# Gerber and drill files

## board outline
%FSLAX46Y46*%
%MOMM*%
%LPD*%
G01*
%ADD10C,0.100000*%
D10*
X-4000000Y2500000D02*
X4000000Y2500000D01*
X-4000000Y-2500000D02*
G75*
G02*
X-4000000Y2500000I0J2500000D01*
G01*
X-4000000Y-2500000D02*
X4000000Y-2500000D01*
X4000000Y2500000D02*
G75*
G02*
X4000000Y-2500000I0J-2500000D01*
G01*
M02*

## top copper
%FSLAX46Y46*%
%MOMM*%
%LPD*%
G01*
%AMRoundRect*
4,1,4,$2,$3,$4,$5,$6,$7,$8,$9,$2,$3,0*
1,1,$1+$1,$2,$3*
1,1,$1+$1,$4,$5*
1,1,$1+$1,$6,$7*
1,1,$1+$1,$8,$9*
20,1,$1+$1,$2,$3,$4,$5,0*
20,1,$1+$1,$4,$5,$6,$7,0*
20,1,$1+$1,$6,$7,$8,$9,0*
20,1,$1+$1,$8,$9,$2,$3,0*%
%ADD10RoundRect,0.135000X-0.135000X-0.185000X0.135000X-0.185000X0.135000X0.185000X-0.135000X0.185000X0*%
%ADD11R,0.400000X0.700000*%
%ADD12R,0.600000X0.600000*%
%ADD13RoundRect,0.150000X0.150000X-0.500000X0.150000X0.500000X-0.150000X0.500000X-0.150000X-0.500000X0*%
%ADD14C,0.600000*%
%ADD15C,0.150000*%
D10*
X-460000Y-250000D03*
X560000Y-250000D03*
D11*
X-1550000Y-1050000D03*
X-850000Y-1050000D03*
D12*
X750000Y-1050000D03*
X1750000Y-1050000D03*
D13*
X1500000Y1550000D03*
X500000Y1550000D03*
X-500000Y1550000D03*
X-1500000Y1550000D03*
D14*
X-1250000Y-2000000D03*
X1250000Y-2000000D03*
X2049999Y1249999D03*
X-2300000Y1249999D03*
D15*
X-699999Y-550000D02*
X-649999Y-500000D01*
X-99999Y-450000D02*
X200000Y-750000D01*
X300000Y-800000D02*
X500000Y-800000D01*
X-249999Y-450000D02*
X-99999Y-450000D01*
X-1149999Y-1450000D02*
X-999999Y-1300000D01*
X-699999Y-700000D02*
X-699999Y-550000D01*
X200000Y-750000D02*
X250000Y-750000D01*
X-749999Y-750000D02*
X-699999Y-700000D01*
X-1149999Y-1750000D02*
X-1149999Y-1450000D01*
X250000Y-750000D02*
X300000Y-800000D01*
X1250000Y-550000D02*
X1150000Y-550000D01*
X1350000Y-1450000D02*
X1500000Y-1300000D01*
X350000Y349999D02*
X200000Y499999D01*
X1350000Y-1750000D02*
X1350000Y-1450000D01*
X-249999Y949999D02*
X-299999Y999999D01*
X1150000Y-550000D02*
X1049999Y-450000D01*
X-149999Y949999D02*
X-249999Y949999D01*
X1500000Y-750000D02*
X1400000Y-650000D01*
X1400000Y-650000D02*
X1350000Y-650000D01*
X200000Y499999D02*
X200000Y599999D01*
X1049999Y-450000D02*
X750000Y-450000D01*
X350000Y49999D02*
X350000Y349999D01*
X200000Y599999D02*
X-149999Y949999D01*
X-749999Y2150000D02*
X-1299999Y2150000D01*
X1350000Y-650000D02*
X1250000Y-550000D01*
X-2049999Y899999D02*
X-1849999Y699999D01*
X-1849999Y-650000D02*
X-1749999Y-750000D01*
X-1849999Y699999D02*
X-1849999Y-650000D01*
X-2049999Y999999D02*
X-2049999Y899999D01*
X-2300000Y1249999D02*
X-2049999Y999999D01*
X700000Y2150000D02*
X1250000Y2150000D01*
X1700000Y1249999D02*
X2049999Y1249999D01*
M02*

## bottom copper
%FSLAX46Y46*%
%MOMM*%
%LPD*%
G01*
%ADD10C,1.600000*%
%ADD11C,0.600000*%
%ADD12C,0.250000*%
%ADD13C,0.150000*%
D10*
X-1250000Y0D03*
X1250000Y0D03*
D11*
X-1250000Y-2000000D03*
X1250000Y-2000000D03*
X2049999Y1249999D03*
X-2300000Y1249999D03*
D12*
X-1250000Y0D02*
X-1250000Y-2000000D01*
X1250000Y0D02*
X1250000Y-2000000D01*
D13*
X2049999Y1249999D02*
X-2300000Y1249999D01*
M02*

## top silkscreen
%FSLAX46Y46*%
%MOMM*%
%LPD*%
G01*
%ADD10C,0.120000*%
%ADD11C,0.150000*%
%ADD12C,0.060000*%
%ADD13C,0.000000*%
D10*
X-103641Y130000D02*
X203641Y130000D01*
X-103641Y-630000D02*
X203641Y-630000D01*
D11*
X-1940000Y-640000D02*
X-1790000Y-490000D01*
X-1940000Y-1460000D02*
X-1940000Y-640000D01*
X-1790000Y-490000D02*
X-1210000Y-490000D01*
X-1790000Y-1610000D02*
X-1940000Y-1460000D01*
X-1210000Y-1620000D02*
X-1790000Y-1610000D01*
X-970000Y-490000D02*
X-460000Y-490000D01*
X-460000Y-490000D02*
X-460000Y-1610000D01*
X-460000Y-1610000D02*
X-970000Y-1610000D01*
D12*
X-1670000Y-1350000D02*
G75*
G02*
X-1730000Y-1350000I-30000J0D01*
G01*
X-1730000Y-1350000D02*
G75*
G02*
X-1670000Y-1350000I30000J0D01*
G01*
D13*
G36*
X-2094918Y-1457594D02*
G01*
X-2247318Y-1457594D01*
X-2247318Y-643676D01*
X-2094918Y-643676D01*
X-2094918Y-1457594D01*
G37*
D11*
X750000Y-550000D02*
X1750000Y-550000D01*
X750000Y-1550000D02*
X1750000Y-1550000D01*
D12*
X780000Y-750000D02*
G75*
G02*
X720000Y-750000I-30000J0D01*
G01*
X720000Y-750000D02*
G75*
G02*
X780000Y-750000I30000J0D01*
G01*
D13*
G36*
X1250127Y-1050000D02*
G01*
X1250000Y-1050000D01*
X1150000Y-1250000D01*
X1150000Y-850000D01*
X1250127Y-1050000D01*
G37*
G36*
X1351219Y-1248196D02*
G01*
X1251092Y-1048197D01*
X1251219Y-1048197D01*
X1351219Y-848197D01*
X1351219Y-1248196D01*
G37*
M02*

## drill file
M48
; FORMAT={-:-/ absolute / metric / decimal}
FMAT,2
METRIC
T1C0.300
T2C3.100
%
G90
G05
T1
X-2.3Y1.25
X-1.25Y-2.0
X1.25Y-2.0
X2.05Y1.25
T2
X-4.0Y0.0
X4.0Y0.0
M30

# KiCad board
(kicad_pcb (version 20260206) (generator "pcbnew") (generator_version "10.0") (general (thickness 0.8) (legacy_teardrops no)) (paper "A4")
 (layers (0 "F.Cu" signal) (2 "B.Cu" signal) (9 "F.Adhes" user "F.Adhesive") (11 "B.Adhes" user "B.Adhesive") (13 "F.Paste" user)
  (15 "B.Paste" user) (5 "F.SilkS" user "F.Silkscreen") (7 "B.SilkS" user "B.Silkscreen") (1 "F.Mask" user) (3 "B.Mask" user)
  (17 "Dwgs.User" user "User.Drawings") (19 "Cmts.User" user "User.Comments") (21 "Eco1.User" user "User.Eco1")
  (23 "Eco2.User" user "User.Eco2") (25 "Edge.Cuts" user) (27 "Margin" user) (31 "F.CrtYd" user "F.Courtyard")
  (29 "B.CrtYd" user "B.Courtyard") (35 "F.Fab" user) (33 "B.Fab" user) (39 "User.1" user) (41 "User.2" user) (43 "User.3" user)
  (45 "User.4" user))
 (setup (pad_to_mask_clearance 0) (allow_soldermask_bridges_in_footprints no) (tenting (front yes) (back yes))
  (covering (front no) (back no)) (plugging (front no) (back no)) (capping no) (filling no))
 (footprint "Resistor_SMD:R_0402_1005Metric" (layer "F.Cu") (at 0.05 0.25)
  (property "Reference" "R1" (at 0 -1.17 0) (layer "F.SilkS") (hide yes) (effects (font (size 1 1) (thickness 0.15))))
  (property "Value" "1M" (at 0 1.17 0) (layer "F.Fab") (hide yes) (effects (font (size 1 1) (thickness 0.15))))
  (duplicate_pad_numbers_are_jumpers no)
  (fp_line (start -0.153641 -0.38) (end 0.153641 -0.38) (stroke (width 0.12) (type solid)) (layer "F.SilkS"))
  (fp_line (start -0.153641 0.38) (end 0.153641 0.38) (stroke (width 0.12) (type solid)) (layer "F.SilkS"))
  (pad "1" smd roundrect (at -0.51 0) (size 0.54 0.64) (layers "F.Cu" "F.Mask" "F.Paste") (roundrect_rratio 0.25) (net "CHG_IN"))
  (pad "2" smd roundrect (at 0.51 0) (size 0.54 0.64) (layers "F.Cu" "F.Mask" "F.Paste") (roundrect_rratio 0.25) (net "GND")))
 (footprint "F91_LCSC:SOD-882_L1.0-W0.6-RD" (layer "F.Cu") (at -1.2 1.05)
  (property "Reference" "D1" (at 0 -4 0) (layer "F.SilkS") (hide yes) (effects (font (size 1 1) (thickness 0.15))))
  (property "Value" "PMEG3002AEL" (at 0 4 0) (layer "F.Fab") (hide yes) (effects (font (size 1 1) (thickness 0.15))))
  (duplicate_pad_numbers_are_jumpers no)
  (fp_line (start -0.74 -0.41) (end -0.59 -0.56) (stroke (width 0.15) (type solid)) (layer "F.SilkS"))
  (fp_line (start -0.74 0.41) (end -0.74 -0.41) (stroke (width 0.15) (type solid)) (layer "F.SilkS"))
  (fp_line (start -0.59 -0.56) (end -0.01 -0.56) (stroke (width 0.15) (type solid)) (layer "F.SilkS"))
  (fp_line (start -0.59 0.56) (end -0.74 0.41) (stroke (width 0.15) (type solid)) (layer "F.SilkS"))
  (fp_line (start -0.01 0.57) (end -0.59 0.56) (stroke (width 0.15) (type solid)) (layer "F.SilkS"))
  (fp_line (start 0.23 -0.56) (end 0.74 -0.56) (stroke (width 0.15) (type solid)) (layer "F.SilkS"))
  (fp_line (start 0.74 -0.56) (end 0.74 0.56) (stroke (width 0.15) (type solid)) (layer "F.SilkS"))
  (fp_line (start 0.74 0.56) (end 0.23 0.56) (stroke (width 0.15) (type solid)) (layer "F.SilkS"))
  (fp_circle (center -0.5 0.3) (end -0.47 0.3) (stroke (width 0.06) (type solid)) (fill no) (layer "F.SilkS"))
  (fp_poly
   (pts (xy -0.894918 0.407594) (xy -0.894918 -0.406324) (xy -1.047318 -0.406324) (xy -1.047318 0.407594) (xy -0.894918 0.407594))
   (stroke (width 0) (type solid)) (fill yes) (layer "F.SilkS"))
  (pad "1" smd rect (at -0.35 0) (size 0.4 0.7) (layers "F.Cu" "F.Mask" "F.Paste") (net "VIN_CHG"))
  (pad "2" smd rect (at 0.35 0) (size 0.4 0.7) (layers "F.Cu" "F.Mask" "F.Paste") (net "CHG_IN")))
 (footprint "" (layer "F.Cu") (at 0 0)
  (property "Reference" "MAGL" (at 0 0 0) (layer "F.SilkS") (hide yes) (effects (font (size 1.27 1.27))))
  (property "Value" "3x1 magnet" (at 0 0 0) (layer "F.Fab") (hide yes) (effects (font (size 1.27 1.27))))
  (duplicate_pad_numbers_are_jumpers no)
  (pad "" np_thru_hole circle (at -4 0) (size 3.1 3.1) (drill 3.1) (layers "*.Cu")))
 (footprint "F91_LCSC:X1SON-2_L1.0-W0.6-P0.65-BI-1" (layer "F.Cu") (at 1.25 1.05)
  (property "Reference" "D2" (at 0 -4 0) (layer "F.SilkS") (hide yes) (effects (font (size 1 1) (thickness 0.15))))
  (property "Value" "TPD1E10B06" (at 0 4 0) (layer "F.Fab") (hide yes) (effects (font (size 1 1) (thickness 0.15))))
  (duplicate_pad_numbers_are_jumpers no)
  (fp_line (start -0.5 -0.5) (end 0.5 -0.5) (stroke (width 0.15) (type solid)) (layer "F.SilkS"))
  (fp_line (start -0.5 0.5) (end 0.5 0.5) (stroke (width 0.15) (type solid)) (layer "F.SilkS"))
  (fp_circle (center -0.5 -0.3) (end -0.47 -0.3) (stroke (width 0.06) (type solid)) (fill no) (layer "F.SilkS"))
  (fp_poly
   (pts (xy -0.1 -0.2) (xy -0.1 0.2) (xy 0 0) (xy 0.000127 0) (xy -0.1 -0.2)) (stroke (width 0) (type solid)) (fill yes) (layer "F.SilkS"))
  (fp_poly
   (pts (xy 0.101219 0.198196) (xy 0.101219 -0.201803) (xy 0.001219 -0.001803) (xy 0.001092 -0.001803) (xy 0.101219 0.198196))
   (stroke (width 0) (type solid)) (fill yes) (layer "F.SilkS"))
  (pad "1" smd rect (at -0.5 0) (size 0.6 0.6) (layers "F.Cu" "F.Mask" "F.Paste") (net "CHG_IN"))
  (pad "2" smd rect (at 0.5 0) (size 0.6 0.6) (layers "F.Cu" "F.Mask" "F.Paste") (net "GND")))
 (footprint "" (layer "F.Cu") (at 0 0)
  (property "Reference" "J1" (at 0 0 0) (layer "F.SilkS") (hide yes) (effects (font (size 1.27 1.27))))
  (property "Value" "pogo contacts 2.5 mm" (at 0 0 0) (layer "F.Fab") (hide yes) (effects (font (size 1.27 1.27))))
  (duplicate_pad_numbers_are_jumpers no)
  (pad "1" smd circle (at -1.25 0) (size 1.6 1.6) (layers "B.Cu" "B.Mask") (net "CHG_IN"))
  (pad "2" smd circle (at 1.25 0) (size 1.6 1.6) (layers "B.Cu" "B.Mask") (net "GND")))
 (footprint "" (layer "F.Cu") (at 0 0)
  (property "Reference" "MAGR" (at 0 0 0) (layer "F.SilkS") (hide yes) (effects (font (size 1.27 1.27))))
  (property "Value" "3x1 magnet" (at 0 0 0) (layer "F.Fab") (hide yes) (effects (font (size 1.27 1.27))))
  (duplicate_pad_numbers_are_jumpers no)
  (pad "" np_thru_hole circle (at 4 0) (size 3.1 3.1) (drill 3.1) (layers "*.Cu")))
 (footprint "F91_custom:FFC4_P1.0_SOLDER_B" (layer "B.Cu") (at 0 -1.55 90)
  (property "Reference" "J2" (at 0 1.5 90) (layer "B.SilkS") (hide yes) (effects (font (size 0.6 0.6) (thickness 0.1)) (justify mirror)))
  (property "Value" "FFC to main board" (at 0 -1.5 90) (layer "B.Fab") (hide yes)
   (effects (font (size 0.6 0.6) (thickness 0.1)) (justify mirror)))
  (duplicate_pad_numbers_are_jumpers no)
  (pad "1" smd roundrect (at 0 1.5 90) (size 1.3 0.6) (layers "F.Cu" "F.Mask") (roundrect_rratio 0.25) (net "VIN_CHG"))
  (pad "2" smd roundrect (at 0 0.5 90) (size 1.3 0.6) (layers "F.Cu" "F.Mask") (roundrect_rratio 0.25) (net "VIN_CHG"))
  (pad "3" smd roundrect (at 0 -0.5 90) (size 1.3 0.6) (layers "F.Cu" "F.Mask") (roundrect_rratio 0.25) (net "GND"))
  (pad "4" smd roundrect (at 0 -1.5 90) (size 1.3 0.6) (layers "F.Cu" "F.Mask") (roundrect_rratio 0.25) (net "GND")))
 (gr_line (start -4 -2.5) (end 4 -2.5) (stroke (width 0.1) (type default)) (layer "Edge.Cuts"))
 (gr_arc (start -4 2.5) (mid -6.5 0) (end -4 -2.5) (stroke (width 0.1) (type default)) (layer "Edge.Cuts"))
 (gr_line (start -4 2.5) (end 4 2.5) (stroke (width 0.1) (type default)) (layer "Edge.Cuts"))
 (gr_arc (start 4 -2.5) (mid 6.5 0) (end 4 2.5) (stroke (width 0.1) (type default)) (layer "Edge.Cuts"))
 (segment (start -0.699999 0.55) (end -0.649999 0.5) (width 0.15) (layer "F.Cu") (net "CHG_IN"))
 (segment (start -0.099999 0.45) (end 0.2 0.75) (width 0.15) (layer "F.Cu") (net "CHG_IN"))
 (segment (start 0.3 0.8) (end 0.5 0.8) (width 0.15) (layer "F.Cu") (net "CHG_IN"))
 (segment (start -0.249999 0.45) (end -0.099999 0.45) (width 0.15) (layer "F.Cu") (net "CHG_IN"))
 (segment (start -1.149999 1.45) (end -0.999999 1.3) (width 0.15) (layer "F.Cu") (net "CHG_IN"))
 (segment (start -0.699999 0.7) (end -0.699999 0.55) (width 0.15) (layer "F.Cu") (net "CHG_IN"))
 (segment (start 0.2 0.75) (end 0.25 0.75) (width 0.15) (layer "F.Cu") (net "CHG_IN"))
 (segment (start -0.749999 0.75) (end -0.699999 0.7) (width 0.15) (layer "F.Cu") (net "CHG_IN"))
 (segment (start -1.149999 1.75) (end -1.149999 1.45) (width 0.15) (layer "F.Cu") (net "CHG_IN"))
 (segment (start 0.25 0.75) (end 0.3 0.8) (width 0.15) (layer "F.Cu") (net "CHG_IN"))
 (via (at -1.25 2) (size 0.6) (drill 0.3) (layers "F.Cu" "B.Cu") (tenting (front yes) (back yes)) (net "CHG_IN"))
 (segment (start -1.25 0) (end -1.25 2) (width 0.25) (layer "B.Cu") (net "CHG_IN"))
 (segment (start 1.25 0.55) (end 1.15 0.55) (width 0.15) (layer "F.Cu") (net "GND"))
 (segment (start 1.35 1.45) (end 1.5 1.3) (width 0.15) (layer "F.Cu") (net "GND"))
 (segment (start 0.35 -0.349999) (end 0.2 -0.499999) (width 0.15) (layer "F.Cu") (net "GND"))
 (segment (start 1.35 1.75) (end 1.35 1.45) (width 0.15) (layer "F.Cu") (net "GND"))
 (segment (start -0.249999 -0.949999) (end -0.299999 -0.999999) (width 0.15) (layer "F.Cu") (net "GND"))
 (segment (start 1.15 0.55) (end 1.049999 0.45) (width 0.15) (layer "F.Cu") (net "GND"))
 (segment (start -0.149999 -0.949999) (end -0.249999 -0.949999) (width 0.15) (layer "F.Cu") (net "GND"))
 (segment (start 1.5 0.75) (end 1.4 0.65) (width 0.15) (layer "F.Cu") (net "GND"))
 (segment (start 1.4 0.65) (end 1.35 0.65) (width 0.15) (layer "F.Cu") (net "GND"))
 (segment (start 0.2 -0.499999) (end 0.2 -0.599999) (width 0.15) (layer "F.Cu") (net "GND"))
 (segment (start 1.049999 0.45) (end 0.75 0.45) (width 0.15) (layer "F.Cu") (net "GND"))
 (segment (start 0.35 -0.049999) (end 0.35 -0.349999) (width 0.15) (layer "F.Cu") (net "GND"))
 (segment (start 0.2 -0.599999) (end -0.149999 -0.949999) (width 0.15) (layer "F.Cu") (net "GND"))
 (segment (start -0.749999 -2.15) (end -1.299999 -2.15) (width 0.15) (layer "F.Cu") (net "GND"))
 (segment (start 1.35 0.65) (end 1.25 0.55) (width 0.15) (layer "F.Cu") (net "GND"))
 (via (at 1.25 2) (size 0.6) (drill 0.3) (layers "F.Cu" "B.Cu") (tenting (front yes) (back yes)) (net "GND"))
 (segment (start 1.25 0) (end 1.25 2) (width 0.25) (layer "B.Cu") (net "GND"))
 (segment (start -2.049999 -0.899999) (end -1.849999 -0.699999) (width 0.15) (layer "F.Cu") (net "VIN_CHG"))
 (segment (start -1.849999 0.65) (end -1.749999 0.75) (width 0.15) (layer "F.Cu") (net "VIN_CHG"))
 (segment (start -1.849999 -0.699999) (end -1.849999 0.65) (width 0.15) (layer "F.Cu") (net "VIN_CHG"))
 (segment (start -2.049999 -0.999999) (end -2.049999 -0.899999) (width 0.15) (layer "F.Cu") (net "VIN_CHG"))
 (segment (start -2.3 -1.249999) (end -2.049999 -0.999999) (width 0.15) (layer "F.Cu") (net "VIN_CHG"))
 (segment (start 0.7 -2.15) (end 1.25 -2.15) (width 0.15) (layer "F.Cu") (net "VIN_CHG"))
 (segment (start 1.7 -1.249999) (end 2.049999 -1.249999) (width 0.15) (layer "F.Cu") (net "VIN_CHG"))
 (via (at 2.049999 -1.249999) (size 0.6) (drill 0.3) (layers "F.Cu" "B.Cu") (tenting (front yes) (back yes)) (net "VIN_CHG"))
 (via (at -2.3 -1.249999) (size 0.6) (drill 0.3) (layers "F.Cu" "B.Cu") (tenting (front yes) (back yes)) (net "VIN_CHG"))
 (segment (start 2.049999 -1.249999) (end -2.3 -1.249999) (width 0.15) (layer "B.Cu") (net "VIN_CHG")))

